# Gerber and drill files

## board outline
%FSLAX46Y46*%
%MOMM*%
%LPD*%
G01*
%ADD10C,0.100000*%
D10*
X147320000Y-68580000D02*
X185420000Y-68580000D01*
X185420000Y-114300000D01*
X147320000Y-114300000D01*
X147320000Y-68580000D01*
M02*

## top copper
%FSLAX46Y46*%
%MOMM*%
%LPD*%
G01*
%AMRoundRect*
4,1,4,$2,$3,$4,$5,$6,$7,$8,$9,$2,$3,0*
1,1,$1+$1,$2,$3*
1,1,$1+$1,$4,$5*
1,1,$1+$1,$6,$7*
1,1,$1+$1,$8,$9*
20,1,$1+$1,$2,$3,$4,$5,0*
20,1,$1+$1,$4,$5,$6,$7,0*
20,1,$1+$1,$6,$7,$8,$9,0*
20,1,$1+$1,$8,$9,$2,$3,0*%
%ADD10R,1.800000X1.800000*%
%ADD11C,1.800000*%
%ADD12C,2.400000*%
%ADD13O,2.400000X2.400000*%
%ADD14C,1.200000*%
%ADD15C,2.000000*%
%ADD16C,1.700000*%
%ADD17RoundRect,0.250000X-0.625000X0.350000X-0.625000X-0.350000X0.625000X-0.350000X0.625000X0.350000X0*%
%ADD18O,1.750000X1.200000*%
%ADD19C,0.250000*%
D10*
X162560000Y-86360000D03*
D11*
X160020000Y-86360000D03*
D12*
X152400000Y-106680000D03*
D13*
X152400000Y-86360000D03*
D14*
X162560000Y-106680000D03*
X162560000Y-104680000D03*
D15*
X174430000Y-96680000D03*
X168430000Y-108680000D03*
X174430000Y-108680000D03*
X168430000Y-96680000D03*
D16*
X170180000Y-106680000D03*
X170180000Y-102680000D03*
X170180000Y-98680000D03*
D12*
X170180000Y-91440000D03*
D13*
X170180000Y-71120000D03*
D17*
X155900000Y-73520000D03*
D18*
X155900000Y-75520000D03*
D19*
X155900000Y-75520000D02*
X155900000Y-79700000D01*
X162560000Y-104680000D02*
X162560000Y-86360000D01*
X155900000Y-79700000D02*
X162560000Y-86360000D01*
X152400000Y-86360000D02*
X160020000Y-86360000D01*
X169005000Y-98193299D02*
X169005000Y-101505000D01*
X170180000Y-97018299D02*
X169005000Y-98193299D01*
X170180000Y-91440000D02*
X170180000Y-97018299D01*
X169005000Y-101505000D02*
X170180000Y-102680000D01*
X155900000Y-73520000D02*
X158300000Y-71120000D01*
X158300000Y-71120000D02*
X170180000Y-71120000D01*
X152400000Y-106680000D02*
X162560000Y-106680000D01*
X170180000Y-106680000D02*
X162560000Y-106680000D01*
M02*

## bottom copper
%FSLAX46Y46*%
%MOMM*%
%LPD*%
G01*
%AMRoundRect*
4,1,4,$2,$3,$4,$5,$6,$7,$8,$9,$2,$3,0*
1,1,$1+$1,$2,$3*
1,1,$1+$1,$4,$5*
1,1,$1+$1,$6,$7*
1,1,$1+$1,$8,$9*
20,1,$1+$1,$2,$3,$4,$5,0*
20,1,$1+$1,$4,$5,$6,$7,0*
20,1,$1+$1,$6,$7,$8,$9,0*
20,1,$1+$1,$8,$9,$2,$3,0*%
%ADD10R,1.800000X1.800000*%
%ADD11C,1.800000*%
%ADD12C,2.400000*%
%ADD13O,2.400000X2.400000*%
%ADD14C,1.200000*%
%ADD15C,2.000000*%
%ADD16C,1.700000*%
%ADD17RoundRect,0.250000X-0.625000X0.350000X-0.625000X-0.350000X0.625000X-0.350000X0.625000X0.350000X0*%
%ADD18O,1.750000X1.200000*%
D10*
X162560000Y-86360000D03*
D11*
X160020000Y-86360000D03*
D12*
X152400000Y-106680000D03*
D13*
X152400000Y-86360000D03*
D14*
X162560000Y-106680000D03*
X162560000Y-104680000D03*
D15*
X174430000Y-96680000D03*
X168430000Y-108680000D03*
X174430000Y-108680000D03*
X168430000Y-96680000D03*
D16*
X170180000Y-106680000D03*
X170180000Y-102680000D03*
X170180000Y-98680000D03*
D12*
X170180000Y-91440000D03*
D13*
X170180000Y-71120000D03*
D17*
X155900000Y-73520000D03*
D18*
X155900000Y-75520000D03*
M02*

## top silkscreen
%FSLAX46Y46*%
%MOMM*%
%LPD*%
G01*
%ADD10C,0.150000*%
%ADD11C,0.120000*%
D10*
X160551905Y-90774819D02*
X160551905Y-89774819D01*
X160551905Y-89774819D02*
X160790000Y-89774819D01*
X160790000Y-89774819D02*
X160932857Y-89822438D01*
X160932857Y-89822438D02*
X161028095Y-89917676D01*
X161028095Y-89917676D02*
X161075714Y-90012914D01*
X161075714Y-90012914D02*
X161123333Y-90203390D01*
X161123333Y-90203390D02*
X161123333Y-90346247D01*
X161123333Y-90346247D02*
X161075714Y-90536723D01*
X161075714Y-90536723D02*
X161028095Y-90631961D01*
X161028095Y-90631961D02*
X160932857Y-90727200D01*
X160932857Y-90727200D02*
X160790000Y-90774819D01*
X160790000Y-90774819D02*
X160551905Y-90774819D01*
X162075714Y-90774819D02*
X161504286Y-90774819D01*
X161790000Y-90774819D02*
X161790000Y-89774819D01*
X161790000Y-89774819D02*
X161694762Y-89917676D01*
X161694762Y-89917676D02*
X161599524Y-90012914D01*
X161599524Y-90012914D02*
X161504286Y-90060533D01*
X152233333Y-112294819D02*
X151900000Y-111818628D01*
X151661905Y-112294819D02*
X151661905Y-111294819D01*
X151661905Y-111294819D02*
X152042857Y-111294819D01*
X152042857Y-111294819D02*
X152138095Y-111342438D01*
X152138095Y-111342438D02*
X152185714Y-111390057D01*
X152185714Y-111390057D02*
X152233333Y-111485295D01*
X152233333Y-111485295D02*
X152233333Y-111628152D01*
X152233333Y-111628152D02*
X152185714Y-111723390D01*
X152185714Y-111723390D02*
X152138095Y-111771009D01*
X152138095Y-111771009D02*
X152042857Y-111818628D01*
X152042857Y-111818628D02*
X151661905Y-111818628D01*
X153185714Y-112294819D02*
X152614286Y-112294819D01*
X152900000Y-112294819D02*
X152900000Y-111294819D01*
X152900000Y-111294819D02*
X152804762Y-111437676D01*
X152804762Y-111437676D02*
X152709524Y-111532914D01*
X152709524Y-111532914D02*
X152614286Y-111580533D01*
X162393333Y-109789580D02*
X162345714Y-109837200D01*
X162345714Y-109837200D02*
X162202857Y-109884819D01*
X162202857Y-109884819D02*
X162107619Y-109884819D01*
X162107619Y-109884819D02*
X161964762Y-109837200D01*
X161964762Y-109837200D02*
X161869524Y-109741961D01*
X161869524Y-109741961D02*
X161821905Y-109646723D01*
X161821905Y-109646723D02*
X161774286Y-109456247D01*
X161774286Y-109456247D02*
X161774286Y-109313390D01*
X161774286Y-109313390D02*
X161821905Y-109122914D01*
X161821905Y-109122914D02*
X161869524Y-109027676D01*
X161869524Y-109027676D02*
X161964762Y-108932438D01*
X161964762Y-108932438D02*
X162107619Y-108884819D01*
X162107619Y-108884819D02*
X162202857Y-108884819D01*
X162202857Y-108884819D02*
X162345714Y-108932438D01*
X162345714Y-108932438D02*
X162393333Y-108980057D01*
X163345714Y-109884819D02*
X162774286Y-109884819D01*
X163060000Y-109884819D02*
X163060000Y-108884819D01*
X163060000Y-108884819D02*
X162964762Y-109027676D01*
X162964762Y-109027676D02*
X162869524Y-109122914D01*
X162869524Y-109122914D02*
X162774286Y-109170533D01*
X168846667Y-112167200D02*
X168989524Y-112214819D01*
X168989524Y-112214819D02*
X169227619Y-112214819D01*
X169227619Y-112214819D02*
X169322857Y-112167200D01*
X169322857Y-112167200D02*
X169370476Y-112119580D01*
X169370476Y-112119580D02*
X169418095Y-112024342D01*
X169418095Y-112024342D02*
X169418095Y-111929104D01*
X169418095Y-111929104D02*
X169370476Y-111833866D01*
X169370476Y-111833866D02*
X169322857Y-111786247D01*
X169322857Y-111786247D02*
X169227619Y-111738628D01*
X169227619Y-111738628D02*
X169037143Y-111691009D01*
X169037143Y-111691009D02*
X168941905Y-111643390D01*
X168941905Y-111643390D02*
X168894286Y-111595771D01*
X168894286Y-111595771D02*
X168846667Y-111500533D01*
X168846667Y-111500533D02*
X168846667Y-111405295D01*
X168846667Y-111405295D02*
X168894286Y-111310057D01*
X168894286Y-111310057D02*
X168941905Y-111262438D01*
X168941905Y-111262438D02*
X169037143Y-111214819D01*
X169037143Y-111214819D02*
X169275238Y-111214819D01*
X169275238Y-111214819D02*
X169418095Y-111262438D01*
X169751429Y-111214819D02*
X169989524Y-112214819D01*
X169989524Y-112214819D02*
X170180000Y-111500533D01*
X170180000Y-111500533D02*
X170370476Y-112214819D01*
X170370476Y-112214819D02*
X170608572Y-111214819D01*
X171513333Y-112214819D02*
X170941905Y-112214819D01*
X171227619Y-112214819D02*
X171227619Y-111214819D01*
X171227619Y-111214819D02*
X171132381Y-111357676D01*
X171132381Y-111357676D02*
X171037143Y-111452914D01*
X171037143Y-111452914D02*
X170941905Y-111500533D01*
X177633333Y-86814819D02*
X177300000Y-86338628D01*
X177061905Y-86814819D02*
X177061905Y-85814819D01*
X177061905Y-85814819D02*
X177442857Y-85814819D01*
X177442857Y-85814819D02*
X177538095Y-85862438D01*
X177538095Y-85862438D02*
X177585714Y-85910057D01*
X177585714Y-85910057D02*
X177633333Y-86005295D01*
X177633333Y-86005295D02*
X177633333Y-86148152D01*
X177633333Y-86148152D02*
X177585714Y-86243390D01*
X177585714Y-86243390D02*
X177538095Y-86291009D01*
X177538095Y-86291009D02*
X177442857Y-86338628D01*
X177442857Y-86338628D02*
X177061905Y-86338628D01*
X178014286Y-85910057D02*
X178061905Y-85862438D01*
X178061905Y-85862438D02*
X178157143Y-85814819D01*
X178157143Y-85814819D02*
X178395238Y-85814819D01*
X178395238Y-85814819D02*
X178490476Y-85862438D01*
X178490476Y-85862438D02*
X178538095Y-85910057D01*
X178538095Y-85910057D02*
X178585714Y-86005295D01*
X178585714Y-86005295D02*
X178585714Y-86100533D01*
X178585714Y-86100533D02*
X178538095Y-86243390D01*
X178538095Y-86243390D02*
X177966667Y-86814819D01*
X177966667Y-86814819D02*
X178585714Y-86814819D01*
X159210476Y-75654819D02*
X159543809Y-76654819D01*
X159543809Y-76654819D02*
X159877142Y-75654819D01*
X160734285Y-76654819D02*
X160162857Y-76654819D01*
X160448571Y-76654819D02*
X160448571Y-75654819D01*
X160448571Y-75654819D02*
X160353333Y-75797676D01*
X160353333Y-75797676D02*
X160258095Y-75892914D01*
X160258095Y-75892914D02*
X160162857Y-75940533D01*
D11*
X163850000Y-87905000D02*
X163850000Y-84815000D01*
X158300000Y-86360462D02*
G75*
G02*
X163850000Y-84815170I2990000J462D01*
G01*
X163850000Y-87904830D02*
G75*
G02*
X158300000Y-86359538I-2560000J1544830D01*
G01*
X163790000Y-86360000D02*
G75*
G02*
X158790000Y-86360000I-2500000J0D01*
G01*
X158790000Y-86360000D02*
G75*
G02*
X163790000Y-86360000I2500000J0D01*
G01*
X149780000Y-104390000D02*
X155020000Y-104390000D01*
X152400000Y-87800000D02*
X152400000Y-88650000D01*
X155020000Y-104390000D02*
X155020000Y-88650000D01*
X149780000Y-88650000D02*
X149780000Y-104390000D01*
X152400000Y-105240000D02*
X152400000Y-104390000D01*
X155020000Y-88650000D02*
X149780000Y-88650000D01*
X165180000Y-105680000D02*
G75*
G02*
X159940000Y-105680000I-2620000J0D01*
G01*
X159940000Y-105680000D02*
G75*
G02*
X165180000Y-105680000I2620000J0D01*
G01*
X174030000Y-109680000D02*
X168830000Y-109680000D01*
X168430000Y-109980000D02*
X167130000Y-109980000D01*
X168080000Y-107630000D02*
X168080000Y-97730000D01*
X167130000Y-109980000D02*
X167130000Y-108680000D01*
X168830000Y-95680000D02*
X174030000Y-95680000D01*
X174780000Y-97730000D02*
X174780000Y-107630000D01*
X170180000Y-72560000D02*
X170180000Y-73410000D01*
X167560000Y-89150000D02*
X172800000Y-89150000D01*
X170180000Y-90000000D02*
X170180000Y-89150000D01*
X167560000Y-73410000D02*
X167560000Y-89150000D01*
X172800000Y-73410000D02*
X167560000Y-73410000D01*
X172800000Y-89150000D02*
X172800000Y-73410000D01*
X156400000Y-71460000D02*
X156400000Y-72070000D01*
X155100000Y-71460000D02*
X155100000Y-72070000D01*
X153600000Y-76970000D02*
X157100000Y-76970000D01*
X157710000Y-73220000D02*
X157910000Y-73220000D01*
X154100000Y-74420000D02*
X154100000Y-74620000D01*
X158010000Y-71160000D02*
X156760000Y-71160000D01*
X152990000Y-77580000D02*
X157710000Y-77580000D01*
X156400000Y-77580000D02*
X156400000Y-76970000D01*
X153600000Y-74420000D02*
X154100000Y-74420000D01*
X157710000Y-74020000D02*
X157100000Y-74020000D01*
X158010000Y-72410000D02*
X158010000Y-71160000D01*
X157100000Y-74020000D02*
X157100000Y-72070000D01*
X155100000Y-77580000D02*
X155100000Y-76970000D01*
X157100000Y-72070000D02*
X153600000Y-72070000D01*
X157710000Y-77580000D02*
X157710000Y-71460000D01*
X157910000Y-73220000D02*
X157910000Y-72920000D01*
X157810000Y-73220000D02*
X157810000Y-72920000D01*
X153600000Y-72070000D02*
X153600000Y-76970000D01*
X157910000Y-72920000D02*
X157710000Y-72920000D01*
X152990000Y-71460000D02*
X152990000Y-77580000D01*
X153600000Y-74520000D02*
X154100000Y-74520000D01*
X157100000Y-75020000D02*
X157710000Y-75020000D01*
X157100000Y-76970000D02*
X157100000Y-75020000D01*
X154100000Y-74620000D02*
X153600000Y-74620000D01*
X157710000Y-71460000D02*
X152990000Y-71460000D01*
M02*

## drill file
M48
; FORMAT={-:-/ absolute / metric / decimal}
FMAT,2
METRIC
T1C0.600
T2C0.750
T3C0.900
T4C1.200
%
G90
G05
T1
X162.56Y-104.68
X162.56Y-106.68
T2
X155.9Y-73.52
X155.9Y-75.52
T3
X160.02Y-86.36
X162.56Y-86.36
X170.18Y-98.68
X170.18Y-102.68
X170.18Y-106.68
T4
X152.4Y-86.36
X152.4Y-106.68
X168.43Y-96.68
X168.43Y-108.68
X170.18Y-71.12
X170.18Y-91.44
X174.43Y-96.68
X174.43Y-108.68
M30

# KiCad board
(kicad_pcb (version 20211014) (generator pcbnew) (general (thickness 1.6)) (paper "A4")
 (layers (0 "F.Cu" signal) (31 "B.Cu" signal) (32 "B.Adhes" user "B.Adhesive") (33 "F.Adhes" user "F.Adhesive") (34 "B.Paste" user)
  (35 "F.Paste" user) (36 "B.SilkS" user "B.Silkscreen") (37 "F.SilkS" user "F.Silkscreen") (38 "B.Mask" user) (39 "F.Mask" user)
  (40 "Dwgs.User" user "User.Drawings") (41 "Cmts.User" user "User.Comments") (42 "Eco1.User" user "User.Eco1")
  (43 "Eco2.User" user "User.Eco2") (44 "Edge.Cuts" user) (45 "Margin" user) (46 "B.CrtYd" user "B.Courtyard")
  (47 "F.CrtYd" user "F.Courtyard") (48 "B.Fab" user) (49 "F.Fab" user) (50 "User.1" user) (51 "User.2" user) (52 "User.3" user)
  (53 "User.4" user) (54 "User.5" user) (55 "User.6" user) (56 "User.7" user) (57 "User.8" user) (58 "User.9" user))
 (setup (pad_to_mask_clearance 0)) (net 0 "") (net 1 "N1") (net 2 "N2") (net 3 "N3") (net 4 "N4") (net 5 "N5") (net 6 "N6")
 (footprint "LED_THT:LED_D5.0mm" (layer "F.Cu") (at 162.56 86.36 180)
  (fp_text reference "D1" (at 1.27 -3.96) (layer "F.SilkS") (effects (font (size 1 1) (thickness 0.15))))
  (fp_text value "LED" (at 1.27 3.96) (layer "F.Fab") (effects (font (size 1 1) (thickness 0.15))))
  (fp_line (start -1.29 -1.545) (end -1.29 1.545) (layer "F.SilkS") (width 0.12))
  (fp_arc (start 4.26 -0.000462) (mid 2.072002 2.880433) (end -1.29 1.54483) (layer "F.SilkS") (width 0.12))
  (fp_arc (start -1.29 -1.54483) (mid 2.072002 -2.880433) (end 4.26 0.000462) (layer "F.SilkS") (width 0.12))
  (fp_circle (center 1.27 0) (end 3.77 0) (layer "F.SilkS") (width 0.12) (fill none))
  (pad "1" thru_hole rect (at 0 0 180) (size 1.8 1.8) (drill 0.9) (layers *.Cu *.Mask) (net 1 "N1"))
  (pad "2" thru_hole circle (at 2.54 0 180) (size 1.8 1.8) (drill 0.9) (layers *.Cu *.Mask) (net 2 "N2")))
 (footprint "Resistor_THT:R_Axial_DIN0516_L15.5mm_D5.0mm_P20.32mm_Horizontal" (layer "F.Cu") (at 152.4 106.68 90)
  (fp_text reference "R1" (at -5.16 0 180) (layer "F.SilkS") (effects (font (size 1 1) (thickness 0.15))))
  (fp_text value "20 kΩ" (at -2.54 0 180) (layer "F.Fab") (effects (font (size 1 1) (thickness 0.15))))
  (fp_line (start 2.29 -2.62) (end 2.29 2.62) (layer "F.SilkS") (width 0.12))
  (fp_line (start 18.88 0) (end 18.03 0) (layer "F.SilkS") (width 0.12))
  (fp_line (start 2.29 2.62) (end 18.03 2.62) (layer "F.SilkS") (width 0.12))
  (fp_line (start 18.03 -2.62) (end 2.29 -2.62) (layer "F.SilkS") (width 0.12))
  (fp_line (start 1.44 0) (end 2.29 0) (layer "F.SilkS") (width 0.12))
  (fp_line (start 18.03 2.62) (end 18.03 -2.62) (layer "F.SilkS") (width 0.12))
  (pad "1" thru_hole circle (at 0 0 90) (size 2.4 2.4) (drill 1.2) (layers *.Cu *.Mask) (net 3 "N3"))
  (pad "2" thru_hole oval (at 20.32 0 90) (size 2.4 2.4) (drill 1.2) (layers *.Cu *.Mask) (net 2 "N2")))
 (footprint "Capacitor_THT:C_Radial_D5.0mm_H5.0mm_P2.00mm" (layer "F.Cu") (at 162.56 106.68 90)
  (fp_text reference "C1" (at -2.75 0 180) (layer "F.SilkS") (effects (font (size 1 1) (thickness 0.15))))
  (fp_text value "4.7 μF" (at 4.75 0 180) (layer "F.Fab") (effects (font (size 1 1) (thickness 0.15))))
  (fp_circle (center 1 0) (end 3.62 0) (layer "F.SilkS") (width 0.12) (fill none))
  (pad "1" thru_hole circle (at 0 0 90) (size 1.2 1.2) (drill 0.6) (layers *.Cu *.Mask) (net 3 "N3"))
  (pad "2" thru_hole circle (at 2 0 90) (size 1.2 1.2) (drill 0.6) (layers *.Cu *.Mask) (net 1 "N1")))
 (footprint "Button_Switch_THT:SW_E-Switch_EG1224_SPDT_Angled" (layer "F.Cu") (at 170.18 106.68 90)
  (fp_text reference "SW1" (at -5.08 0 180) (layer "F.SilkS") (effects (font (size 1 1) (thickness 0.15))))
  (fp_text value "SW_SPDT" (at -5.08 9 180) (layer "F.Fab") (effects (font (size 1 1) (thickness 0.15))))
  (fp_line (start -3 3.85) (end -3 -1.35) (layer "F.SilkS") (width 0.12))
  (fp_line (start -3.3 -1.75) (end -3.3 -3.05) (layer "F.SilkS") (width 0.12))
  (fp_line (start -0.95 -2.1) (end 8.95 -2.1) (layer "F.SilkS") (width 0.12))
  (fp_line (start -3.3 -3.05) (end -2 -3.05) (layer "F.SilkS") (width 0.12))
  (fp_line (start 11 -1.35) (end 11 3.85) (layer "F.SilkS") (width 0.12))
  (fp_line (start 8.95 4.6) (end -0.95 4.6) (layer "F.SilkS") (width 0.12))
  (pad "" thru_hole circle (at 10 4.25 90) (size 2 2) (drill 1.2) (layers *.Cu *.Mask))
  (pad "" thru_hole circle (at -2 -1.75 90) (size 2 2) (drill 1.2) (layers *.Cu *.Mask))
  (pad "" thru_hole circle (at -2 4.25 90) (size 2 2) (drill 1.2) (layers *.Cu *.Mask))
  (pad "" thru_hole circle (at 10 -1.75 90) (size 2 2) (drill 1.2) (layers *.Cu *.Mask))
  (pad "1" thru_hole circle (at 0 0 90) (size 1.7 1.7) (drill 0.9) (layers *.Cu *.Mask) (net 3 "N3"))
  (pad "2" thru_hole circle (at 4 0 90) (size 1.7 1.7) (drill 0.9) (layers *.Cu *.Mask) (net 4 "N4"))
  (pad "3" thru_hole circle (at 8 0 90) (size 1.7 1.7) (drill 0.9) (layers *.Cu *.Mask) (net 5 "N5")))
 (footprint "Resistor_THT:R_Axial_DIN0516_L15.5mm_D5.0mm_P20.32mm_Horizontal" (layer "F.Cu") (at 170.18 91.44 90)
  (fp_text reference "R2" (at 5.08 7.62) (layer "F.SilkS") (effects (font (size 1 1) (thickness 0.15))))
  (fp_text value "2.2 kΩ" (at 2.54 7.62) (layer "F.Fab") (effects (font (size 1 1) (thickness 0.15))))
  (fp_line (start 18.88 0) (end 18.03 0) (layer "F.SilkS") (width 0.12))
  (fp_line (start 2.29 -2.62) (end 2.29 2.62) (layer "F.SilkS") (width 0.12))
  (fp_line (start 1.44 0) (end 2.29 0) (layer "F.SilkS") (width 0.12))
  (fp_line (start 18.03 -2.62) (end 2.29 -2.62) (layer "F.SilkS") (width 0.12))
  (fp_line (start 18.03 2.62) (end 18.03 -2.62) (layer "F.SilkS") (width 0.12))
  (fp_line (start 2.29 2.62) (end 18.03 2.62) (layer "F.SilkS") (width 0.12))
  (pad "1" thru_hole circle (at 0 0 90) (size 2.4 2.4) (drill 1.2) (layers *.Cu *.Mask) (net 4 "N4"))
  (pad "2" thru_hole oval (at 20.32 0 90) (size 2.4 2.4) (drill 1.2) (layers *.Cu *.Mask) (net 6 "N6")))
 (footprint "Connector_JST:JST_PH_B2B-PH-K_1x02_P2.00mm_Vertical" (layer "F.Cu") (at 155.9 73.52 -90)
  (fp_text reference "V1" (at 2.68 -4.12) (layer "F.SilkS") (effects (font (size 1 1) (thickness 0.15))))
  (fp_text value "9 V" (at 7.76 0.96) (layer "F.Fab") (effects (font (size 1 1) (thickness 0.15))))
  (fp_line (start -2.06 -0.5) (end -1.45 -0.5) (layer "F.SilkS") (width 0.12))
  (fp_line (start -2.06 0.8) (end -1.45 0.8) (layer "F.SilkS") (width 0.12))
  (fp_line (start 3.45 2.3) (end 3.45 -1.2) (layer "F.SilkS") (width 0.12))
  (fp_line (start -0.3 -1.81) (end -0.3 -2.01) (layer "F.SilkS") (width 0.12))
  (fp_line (start 0.9 1.8) (end 1.1 1.8) (layer "F.SilkS") (width 0.12))
  (fp_line (start -2.36 -2.11) (end -2.36 -0.86) (layer "F.SilkS") (width 0.12))
  (fp_line (start 4.06 2.91) (end 4.06 -1.81) (layer "F.SilkS") (width 0.12))
  (fp_line (start 4.06 -0.5) (end 3.45 -0.5) (layer "F.SilkS") (width 0.12))
  (fp_line (start 0.9 2.3) (end 0.9 1.8) (layer "F.SilkS") (width 0.12))
  (fp_line (start 0.5 -1.81) (end 0.5 -1.2) (layer "F.SilkS") (width 0.12))
  (fp_line (start -1.11 -2.11) (end -2.36 -2.11) (layer "F.SilkS") (width 0.12))
  (fp_line (start 0.5 -1.2) (end -1.45 -1.2) (layer "F.SilkS") (width 0.12))
  (fp_line (start 4.06 0.8) (end 3.45 0.8) (layer "F.SilkS") (width 0.12))
  (fp_line (start -1.45 -1.2) (end -1.45 2.3) (layer "F.SilkS") (width 0.12))
  (fp_line (start 4.06 -1.81) (end -2.06 -1.81) (layer "F.SilkS") (width 0.12))
  (fp_line (start -0.3 -2.01) (end -0.6 -2.01) (layer "F.SilkS") (width 0.12))
  (fp_line (start -0.3 -1.91) (end -0.6 -1.91) (layer "F.SilkS") (width 0.12))
  (fp_line (start -1.45 2.3) (end 3.45 2.3) (layer "F.SilkS") (width 0.12))
  (fp_line (start -0.6 -2.01) (end -0.6 -1.81) (layer "F.SilkS") (width 0.12))
  (fp_line (start -2.06 2.91) (end 4.06 2.91) (layer "F.SilkS") (width 0.12))
  (fp_line (start 1 2.3) (end 1 1.8) (layer "F.SilkS") (width 0.12))
  (fp_line (start 1.5 -1.2) (end 1.5 -1.81) (layer "F.SilkS") (width 0.12))
  (fp_line (start 3.45 -1.2) (end 1.5 -1.2) (layer "F.SilkS") (width 0.12))
  (fp_line (start 1.1 1.8) (end 1.1 2.3) (layer "F.SilkS") (width 0.12))
  (fp_line (start -2.06 -1.81) (end -2.06 2.91) (layer "F.SilkS") (width 0.12))
  (pad "1" thru_hole roundrect (at 0 0 270) (size 1.2 1.75) (drill 0.75) (layers *.Cu *.Mask) (roundrect_rratio 0.208333) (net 6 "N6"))
  (pad "2" thru_hole oval (at 2 0 270) (size 1.2 1.75) (drill 0.75) (layers *.Cu *.Mask) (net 1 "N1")))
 (gr_rect (start 147.32 68.58) (end 185.42 114.3) (layer "Edge.Cuts") (width 0.1) (fill none))
 (segment (start 155.9 75.52) (end 155.9 79.7) (width 0.25) (layer "F.Cu") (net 1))
 (segment (start 162.56 104.68) (end 162.56 86.36) (width 0.25) (layer "F.Cu") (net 1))
 (segment (start 155.9 79.7) (end 162.56 86.36) (width 0.25) (layer "F.Cu") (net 1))
 (segment (start 152.4 86.36) (end 160.02 86.36) (width 0.25) (layer "F.Cu") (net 2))
 (segment (start 169.005 98.193299) (end 169.005 101.505) (width 0.25) (layer "F.Cu") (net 4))
 (segment (start 170.18 97.018299) (end 169.005 98.193299) (width 0.25) (layer "F.Cu") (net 4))
 (segment (start 170.18 91.44) (end 170.18 97.018299) (width 0.25) (layer "F.Cu") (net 4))
 (segment (start 169.005 101.505) (end 170.18 102.68) (width 0.25) (layer "F.Cu") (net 4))
 (segment (start 155.9 73.52) (end 158.3 71.12) (width 0.25) (layer "F.Cu") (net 6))
 (segment (start 158.3 71.12) (end 170.18 71.12) (width 0.25) (layer "F.Cu") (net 6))
 (segment (start 152.4 106.68) (end 162.56 106.68) (width 0.25) (layer "F.Cu") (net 3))
 (segment (start 170.18 106.68) (end 162.56 106.68) (width 0.25) (layer "F.Cu") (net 3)))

